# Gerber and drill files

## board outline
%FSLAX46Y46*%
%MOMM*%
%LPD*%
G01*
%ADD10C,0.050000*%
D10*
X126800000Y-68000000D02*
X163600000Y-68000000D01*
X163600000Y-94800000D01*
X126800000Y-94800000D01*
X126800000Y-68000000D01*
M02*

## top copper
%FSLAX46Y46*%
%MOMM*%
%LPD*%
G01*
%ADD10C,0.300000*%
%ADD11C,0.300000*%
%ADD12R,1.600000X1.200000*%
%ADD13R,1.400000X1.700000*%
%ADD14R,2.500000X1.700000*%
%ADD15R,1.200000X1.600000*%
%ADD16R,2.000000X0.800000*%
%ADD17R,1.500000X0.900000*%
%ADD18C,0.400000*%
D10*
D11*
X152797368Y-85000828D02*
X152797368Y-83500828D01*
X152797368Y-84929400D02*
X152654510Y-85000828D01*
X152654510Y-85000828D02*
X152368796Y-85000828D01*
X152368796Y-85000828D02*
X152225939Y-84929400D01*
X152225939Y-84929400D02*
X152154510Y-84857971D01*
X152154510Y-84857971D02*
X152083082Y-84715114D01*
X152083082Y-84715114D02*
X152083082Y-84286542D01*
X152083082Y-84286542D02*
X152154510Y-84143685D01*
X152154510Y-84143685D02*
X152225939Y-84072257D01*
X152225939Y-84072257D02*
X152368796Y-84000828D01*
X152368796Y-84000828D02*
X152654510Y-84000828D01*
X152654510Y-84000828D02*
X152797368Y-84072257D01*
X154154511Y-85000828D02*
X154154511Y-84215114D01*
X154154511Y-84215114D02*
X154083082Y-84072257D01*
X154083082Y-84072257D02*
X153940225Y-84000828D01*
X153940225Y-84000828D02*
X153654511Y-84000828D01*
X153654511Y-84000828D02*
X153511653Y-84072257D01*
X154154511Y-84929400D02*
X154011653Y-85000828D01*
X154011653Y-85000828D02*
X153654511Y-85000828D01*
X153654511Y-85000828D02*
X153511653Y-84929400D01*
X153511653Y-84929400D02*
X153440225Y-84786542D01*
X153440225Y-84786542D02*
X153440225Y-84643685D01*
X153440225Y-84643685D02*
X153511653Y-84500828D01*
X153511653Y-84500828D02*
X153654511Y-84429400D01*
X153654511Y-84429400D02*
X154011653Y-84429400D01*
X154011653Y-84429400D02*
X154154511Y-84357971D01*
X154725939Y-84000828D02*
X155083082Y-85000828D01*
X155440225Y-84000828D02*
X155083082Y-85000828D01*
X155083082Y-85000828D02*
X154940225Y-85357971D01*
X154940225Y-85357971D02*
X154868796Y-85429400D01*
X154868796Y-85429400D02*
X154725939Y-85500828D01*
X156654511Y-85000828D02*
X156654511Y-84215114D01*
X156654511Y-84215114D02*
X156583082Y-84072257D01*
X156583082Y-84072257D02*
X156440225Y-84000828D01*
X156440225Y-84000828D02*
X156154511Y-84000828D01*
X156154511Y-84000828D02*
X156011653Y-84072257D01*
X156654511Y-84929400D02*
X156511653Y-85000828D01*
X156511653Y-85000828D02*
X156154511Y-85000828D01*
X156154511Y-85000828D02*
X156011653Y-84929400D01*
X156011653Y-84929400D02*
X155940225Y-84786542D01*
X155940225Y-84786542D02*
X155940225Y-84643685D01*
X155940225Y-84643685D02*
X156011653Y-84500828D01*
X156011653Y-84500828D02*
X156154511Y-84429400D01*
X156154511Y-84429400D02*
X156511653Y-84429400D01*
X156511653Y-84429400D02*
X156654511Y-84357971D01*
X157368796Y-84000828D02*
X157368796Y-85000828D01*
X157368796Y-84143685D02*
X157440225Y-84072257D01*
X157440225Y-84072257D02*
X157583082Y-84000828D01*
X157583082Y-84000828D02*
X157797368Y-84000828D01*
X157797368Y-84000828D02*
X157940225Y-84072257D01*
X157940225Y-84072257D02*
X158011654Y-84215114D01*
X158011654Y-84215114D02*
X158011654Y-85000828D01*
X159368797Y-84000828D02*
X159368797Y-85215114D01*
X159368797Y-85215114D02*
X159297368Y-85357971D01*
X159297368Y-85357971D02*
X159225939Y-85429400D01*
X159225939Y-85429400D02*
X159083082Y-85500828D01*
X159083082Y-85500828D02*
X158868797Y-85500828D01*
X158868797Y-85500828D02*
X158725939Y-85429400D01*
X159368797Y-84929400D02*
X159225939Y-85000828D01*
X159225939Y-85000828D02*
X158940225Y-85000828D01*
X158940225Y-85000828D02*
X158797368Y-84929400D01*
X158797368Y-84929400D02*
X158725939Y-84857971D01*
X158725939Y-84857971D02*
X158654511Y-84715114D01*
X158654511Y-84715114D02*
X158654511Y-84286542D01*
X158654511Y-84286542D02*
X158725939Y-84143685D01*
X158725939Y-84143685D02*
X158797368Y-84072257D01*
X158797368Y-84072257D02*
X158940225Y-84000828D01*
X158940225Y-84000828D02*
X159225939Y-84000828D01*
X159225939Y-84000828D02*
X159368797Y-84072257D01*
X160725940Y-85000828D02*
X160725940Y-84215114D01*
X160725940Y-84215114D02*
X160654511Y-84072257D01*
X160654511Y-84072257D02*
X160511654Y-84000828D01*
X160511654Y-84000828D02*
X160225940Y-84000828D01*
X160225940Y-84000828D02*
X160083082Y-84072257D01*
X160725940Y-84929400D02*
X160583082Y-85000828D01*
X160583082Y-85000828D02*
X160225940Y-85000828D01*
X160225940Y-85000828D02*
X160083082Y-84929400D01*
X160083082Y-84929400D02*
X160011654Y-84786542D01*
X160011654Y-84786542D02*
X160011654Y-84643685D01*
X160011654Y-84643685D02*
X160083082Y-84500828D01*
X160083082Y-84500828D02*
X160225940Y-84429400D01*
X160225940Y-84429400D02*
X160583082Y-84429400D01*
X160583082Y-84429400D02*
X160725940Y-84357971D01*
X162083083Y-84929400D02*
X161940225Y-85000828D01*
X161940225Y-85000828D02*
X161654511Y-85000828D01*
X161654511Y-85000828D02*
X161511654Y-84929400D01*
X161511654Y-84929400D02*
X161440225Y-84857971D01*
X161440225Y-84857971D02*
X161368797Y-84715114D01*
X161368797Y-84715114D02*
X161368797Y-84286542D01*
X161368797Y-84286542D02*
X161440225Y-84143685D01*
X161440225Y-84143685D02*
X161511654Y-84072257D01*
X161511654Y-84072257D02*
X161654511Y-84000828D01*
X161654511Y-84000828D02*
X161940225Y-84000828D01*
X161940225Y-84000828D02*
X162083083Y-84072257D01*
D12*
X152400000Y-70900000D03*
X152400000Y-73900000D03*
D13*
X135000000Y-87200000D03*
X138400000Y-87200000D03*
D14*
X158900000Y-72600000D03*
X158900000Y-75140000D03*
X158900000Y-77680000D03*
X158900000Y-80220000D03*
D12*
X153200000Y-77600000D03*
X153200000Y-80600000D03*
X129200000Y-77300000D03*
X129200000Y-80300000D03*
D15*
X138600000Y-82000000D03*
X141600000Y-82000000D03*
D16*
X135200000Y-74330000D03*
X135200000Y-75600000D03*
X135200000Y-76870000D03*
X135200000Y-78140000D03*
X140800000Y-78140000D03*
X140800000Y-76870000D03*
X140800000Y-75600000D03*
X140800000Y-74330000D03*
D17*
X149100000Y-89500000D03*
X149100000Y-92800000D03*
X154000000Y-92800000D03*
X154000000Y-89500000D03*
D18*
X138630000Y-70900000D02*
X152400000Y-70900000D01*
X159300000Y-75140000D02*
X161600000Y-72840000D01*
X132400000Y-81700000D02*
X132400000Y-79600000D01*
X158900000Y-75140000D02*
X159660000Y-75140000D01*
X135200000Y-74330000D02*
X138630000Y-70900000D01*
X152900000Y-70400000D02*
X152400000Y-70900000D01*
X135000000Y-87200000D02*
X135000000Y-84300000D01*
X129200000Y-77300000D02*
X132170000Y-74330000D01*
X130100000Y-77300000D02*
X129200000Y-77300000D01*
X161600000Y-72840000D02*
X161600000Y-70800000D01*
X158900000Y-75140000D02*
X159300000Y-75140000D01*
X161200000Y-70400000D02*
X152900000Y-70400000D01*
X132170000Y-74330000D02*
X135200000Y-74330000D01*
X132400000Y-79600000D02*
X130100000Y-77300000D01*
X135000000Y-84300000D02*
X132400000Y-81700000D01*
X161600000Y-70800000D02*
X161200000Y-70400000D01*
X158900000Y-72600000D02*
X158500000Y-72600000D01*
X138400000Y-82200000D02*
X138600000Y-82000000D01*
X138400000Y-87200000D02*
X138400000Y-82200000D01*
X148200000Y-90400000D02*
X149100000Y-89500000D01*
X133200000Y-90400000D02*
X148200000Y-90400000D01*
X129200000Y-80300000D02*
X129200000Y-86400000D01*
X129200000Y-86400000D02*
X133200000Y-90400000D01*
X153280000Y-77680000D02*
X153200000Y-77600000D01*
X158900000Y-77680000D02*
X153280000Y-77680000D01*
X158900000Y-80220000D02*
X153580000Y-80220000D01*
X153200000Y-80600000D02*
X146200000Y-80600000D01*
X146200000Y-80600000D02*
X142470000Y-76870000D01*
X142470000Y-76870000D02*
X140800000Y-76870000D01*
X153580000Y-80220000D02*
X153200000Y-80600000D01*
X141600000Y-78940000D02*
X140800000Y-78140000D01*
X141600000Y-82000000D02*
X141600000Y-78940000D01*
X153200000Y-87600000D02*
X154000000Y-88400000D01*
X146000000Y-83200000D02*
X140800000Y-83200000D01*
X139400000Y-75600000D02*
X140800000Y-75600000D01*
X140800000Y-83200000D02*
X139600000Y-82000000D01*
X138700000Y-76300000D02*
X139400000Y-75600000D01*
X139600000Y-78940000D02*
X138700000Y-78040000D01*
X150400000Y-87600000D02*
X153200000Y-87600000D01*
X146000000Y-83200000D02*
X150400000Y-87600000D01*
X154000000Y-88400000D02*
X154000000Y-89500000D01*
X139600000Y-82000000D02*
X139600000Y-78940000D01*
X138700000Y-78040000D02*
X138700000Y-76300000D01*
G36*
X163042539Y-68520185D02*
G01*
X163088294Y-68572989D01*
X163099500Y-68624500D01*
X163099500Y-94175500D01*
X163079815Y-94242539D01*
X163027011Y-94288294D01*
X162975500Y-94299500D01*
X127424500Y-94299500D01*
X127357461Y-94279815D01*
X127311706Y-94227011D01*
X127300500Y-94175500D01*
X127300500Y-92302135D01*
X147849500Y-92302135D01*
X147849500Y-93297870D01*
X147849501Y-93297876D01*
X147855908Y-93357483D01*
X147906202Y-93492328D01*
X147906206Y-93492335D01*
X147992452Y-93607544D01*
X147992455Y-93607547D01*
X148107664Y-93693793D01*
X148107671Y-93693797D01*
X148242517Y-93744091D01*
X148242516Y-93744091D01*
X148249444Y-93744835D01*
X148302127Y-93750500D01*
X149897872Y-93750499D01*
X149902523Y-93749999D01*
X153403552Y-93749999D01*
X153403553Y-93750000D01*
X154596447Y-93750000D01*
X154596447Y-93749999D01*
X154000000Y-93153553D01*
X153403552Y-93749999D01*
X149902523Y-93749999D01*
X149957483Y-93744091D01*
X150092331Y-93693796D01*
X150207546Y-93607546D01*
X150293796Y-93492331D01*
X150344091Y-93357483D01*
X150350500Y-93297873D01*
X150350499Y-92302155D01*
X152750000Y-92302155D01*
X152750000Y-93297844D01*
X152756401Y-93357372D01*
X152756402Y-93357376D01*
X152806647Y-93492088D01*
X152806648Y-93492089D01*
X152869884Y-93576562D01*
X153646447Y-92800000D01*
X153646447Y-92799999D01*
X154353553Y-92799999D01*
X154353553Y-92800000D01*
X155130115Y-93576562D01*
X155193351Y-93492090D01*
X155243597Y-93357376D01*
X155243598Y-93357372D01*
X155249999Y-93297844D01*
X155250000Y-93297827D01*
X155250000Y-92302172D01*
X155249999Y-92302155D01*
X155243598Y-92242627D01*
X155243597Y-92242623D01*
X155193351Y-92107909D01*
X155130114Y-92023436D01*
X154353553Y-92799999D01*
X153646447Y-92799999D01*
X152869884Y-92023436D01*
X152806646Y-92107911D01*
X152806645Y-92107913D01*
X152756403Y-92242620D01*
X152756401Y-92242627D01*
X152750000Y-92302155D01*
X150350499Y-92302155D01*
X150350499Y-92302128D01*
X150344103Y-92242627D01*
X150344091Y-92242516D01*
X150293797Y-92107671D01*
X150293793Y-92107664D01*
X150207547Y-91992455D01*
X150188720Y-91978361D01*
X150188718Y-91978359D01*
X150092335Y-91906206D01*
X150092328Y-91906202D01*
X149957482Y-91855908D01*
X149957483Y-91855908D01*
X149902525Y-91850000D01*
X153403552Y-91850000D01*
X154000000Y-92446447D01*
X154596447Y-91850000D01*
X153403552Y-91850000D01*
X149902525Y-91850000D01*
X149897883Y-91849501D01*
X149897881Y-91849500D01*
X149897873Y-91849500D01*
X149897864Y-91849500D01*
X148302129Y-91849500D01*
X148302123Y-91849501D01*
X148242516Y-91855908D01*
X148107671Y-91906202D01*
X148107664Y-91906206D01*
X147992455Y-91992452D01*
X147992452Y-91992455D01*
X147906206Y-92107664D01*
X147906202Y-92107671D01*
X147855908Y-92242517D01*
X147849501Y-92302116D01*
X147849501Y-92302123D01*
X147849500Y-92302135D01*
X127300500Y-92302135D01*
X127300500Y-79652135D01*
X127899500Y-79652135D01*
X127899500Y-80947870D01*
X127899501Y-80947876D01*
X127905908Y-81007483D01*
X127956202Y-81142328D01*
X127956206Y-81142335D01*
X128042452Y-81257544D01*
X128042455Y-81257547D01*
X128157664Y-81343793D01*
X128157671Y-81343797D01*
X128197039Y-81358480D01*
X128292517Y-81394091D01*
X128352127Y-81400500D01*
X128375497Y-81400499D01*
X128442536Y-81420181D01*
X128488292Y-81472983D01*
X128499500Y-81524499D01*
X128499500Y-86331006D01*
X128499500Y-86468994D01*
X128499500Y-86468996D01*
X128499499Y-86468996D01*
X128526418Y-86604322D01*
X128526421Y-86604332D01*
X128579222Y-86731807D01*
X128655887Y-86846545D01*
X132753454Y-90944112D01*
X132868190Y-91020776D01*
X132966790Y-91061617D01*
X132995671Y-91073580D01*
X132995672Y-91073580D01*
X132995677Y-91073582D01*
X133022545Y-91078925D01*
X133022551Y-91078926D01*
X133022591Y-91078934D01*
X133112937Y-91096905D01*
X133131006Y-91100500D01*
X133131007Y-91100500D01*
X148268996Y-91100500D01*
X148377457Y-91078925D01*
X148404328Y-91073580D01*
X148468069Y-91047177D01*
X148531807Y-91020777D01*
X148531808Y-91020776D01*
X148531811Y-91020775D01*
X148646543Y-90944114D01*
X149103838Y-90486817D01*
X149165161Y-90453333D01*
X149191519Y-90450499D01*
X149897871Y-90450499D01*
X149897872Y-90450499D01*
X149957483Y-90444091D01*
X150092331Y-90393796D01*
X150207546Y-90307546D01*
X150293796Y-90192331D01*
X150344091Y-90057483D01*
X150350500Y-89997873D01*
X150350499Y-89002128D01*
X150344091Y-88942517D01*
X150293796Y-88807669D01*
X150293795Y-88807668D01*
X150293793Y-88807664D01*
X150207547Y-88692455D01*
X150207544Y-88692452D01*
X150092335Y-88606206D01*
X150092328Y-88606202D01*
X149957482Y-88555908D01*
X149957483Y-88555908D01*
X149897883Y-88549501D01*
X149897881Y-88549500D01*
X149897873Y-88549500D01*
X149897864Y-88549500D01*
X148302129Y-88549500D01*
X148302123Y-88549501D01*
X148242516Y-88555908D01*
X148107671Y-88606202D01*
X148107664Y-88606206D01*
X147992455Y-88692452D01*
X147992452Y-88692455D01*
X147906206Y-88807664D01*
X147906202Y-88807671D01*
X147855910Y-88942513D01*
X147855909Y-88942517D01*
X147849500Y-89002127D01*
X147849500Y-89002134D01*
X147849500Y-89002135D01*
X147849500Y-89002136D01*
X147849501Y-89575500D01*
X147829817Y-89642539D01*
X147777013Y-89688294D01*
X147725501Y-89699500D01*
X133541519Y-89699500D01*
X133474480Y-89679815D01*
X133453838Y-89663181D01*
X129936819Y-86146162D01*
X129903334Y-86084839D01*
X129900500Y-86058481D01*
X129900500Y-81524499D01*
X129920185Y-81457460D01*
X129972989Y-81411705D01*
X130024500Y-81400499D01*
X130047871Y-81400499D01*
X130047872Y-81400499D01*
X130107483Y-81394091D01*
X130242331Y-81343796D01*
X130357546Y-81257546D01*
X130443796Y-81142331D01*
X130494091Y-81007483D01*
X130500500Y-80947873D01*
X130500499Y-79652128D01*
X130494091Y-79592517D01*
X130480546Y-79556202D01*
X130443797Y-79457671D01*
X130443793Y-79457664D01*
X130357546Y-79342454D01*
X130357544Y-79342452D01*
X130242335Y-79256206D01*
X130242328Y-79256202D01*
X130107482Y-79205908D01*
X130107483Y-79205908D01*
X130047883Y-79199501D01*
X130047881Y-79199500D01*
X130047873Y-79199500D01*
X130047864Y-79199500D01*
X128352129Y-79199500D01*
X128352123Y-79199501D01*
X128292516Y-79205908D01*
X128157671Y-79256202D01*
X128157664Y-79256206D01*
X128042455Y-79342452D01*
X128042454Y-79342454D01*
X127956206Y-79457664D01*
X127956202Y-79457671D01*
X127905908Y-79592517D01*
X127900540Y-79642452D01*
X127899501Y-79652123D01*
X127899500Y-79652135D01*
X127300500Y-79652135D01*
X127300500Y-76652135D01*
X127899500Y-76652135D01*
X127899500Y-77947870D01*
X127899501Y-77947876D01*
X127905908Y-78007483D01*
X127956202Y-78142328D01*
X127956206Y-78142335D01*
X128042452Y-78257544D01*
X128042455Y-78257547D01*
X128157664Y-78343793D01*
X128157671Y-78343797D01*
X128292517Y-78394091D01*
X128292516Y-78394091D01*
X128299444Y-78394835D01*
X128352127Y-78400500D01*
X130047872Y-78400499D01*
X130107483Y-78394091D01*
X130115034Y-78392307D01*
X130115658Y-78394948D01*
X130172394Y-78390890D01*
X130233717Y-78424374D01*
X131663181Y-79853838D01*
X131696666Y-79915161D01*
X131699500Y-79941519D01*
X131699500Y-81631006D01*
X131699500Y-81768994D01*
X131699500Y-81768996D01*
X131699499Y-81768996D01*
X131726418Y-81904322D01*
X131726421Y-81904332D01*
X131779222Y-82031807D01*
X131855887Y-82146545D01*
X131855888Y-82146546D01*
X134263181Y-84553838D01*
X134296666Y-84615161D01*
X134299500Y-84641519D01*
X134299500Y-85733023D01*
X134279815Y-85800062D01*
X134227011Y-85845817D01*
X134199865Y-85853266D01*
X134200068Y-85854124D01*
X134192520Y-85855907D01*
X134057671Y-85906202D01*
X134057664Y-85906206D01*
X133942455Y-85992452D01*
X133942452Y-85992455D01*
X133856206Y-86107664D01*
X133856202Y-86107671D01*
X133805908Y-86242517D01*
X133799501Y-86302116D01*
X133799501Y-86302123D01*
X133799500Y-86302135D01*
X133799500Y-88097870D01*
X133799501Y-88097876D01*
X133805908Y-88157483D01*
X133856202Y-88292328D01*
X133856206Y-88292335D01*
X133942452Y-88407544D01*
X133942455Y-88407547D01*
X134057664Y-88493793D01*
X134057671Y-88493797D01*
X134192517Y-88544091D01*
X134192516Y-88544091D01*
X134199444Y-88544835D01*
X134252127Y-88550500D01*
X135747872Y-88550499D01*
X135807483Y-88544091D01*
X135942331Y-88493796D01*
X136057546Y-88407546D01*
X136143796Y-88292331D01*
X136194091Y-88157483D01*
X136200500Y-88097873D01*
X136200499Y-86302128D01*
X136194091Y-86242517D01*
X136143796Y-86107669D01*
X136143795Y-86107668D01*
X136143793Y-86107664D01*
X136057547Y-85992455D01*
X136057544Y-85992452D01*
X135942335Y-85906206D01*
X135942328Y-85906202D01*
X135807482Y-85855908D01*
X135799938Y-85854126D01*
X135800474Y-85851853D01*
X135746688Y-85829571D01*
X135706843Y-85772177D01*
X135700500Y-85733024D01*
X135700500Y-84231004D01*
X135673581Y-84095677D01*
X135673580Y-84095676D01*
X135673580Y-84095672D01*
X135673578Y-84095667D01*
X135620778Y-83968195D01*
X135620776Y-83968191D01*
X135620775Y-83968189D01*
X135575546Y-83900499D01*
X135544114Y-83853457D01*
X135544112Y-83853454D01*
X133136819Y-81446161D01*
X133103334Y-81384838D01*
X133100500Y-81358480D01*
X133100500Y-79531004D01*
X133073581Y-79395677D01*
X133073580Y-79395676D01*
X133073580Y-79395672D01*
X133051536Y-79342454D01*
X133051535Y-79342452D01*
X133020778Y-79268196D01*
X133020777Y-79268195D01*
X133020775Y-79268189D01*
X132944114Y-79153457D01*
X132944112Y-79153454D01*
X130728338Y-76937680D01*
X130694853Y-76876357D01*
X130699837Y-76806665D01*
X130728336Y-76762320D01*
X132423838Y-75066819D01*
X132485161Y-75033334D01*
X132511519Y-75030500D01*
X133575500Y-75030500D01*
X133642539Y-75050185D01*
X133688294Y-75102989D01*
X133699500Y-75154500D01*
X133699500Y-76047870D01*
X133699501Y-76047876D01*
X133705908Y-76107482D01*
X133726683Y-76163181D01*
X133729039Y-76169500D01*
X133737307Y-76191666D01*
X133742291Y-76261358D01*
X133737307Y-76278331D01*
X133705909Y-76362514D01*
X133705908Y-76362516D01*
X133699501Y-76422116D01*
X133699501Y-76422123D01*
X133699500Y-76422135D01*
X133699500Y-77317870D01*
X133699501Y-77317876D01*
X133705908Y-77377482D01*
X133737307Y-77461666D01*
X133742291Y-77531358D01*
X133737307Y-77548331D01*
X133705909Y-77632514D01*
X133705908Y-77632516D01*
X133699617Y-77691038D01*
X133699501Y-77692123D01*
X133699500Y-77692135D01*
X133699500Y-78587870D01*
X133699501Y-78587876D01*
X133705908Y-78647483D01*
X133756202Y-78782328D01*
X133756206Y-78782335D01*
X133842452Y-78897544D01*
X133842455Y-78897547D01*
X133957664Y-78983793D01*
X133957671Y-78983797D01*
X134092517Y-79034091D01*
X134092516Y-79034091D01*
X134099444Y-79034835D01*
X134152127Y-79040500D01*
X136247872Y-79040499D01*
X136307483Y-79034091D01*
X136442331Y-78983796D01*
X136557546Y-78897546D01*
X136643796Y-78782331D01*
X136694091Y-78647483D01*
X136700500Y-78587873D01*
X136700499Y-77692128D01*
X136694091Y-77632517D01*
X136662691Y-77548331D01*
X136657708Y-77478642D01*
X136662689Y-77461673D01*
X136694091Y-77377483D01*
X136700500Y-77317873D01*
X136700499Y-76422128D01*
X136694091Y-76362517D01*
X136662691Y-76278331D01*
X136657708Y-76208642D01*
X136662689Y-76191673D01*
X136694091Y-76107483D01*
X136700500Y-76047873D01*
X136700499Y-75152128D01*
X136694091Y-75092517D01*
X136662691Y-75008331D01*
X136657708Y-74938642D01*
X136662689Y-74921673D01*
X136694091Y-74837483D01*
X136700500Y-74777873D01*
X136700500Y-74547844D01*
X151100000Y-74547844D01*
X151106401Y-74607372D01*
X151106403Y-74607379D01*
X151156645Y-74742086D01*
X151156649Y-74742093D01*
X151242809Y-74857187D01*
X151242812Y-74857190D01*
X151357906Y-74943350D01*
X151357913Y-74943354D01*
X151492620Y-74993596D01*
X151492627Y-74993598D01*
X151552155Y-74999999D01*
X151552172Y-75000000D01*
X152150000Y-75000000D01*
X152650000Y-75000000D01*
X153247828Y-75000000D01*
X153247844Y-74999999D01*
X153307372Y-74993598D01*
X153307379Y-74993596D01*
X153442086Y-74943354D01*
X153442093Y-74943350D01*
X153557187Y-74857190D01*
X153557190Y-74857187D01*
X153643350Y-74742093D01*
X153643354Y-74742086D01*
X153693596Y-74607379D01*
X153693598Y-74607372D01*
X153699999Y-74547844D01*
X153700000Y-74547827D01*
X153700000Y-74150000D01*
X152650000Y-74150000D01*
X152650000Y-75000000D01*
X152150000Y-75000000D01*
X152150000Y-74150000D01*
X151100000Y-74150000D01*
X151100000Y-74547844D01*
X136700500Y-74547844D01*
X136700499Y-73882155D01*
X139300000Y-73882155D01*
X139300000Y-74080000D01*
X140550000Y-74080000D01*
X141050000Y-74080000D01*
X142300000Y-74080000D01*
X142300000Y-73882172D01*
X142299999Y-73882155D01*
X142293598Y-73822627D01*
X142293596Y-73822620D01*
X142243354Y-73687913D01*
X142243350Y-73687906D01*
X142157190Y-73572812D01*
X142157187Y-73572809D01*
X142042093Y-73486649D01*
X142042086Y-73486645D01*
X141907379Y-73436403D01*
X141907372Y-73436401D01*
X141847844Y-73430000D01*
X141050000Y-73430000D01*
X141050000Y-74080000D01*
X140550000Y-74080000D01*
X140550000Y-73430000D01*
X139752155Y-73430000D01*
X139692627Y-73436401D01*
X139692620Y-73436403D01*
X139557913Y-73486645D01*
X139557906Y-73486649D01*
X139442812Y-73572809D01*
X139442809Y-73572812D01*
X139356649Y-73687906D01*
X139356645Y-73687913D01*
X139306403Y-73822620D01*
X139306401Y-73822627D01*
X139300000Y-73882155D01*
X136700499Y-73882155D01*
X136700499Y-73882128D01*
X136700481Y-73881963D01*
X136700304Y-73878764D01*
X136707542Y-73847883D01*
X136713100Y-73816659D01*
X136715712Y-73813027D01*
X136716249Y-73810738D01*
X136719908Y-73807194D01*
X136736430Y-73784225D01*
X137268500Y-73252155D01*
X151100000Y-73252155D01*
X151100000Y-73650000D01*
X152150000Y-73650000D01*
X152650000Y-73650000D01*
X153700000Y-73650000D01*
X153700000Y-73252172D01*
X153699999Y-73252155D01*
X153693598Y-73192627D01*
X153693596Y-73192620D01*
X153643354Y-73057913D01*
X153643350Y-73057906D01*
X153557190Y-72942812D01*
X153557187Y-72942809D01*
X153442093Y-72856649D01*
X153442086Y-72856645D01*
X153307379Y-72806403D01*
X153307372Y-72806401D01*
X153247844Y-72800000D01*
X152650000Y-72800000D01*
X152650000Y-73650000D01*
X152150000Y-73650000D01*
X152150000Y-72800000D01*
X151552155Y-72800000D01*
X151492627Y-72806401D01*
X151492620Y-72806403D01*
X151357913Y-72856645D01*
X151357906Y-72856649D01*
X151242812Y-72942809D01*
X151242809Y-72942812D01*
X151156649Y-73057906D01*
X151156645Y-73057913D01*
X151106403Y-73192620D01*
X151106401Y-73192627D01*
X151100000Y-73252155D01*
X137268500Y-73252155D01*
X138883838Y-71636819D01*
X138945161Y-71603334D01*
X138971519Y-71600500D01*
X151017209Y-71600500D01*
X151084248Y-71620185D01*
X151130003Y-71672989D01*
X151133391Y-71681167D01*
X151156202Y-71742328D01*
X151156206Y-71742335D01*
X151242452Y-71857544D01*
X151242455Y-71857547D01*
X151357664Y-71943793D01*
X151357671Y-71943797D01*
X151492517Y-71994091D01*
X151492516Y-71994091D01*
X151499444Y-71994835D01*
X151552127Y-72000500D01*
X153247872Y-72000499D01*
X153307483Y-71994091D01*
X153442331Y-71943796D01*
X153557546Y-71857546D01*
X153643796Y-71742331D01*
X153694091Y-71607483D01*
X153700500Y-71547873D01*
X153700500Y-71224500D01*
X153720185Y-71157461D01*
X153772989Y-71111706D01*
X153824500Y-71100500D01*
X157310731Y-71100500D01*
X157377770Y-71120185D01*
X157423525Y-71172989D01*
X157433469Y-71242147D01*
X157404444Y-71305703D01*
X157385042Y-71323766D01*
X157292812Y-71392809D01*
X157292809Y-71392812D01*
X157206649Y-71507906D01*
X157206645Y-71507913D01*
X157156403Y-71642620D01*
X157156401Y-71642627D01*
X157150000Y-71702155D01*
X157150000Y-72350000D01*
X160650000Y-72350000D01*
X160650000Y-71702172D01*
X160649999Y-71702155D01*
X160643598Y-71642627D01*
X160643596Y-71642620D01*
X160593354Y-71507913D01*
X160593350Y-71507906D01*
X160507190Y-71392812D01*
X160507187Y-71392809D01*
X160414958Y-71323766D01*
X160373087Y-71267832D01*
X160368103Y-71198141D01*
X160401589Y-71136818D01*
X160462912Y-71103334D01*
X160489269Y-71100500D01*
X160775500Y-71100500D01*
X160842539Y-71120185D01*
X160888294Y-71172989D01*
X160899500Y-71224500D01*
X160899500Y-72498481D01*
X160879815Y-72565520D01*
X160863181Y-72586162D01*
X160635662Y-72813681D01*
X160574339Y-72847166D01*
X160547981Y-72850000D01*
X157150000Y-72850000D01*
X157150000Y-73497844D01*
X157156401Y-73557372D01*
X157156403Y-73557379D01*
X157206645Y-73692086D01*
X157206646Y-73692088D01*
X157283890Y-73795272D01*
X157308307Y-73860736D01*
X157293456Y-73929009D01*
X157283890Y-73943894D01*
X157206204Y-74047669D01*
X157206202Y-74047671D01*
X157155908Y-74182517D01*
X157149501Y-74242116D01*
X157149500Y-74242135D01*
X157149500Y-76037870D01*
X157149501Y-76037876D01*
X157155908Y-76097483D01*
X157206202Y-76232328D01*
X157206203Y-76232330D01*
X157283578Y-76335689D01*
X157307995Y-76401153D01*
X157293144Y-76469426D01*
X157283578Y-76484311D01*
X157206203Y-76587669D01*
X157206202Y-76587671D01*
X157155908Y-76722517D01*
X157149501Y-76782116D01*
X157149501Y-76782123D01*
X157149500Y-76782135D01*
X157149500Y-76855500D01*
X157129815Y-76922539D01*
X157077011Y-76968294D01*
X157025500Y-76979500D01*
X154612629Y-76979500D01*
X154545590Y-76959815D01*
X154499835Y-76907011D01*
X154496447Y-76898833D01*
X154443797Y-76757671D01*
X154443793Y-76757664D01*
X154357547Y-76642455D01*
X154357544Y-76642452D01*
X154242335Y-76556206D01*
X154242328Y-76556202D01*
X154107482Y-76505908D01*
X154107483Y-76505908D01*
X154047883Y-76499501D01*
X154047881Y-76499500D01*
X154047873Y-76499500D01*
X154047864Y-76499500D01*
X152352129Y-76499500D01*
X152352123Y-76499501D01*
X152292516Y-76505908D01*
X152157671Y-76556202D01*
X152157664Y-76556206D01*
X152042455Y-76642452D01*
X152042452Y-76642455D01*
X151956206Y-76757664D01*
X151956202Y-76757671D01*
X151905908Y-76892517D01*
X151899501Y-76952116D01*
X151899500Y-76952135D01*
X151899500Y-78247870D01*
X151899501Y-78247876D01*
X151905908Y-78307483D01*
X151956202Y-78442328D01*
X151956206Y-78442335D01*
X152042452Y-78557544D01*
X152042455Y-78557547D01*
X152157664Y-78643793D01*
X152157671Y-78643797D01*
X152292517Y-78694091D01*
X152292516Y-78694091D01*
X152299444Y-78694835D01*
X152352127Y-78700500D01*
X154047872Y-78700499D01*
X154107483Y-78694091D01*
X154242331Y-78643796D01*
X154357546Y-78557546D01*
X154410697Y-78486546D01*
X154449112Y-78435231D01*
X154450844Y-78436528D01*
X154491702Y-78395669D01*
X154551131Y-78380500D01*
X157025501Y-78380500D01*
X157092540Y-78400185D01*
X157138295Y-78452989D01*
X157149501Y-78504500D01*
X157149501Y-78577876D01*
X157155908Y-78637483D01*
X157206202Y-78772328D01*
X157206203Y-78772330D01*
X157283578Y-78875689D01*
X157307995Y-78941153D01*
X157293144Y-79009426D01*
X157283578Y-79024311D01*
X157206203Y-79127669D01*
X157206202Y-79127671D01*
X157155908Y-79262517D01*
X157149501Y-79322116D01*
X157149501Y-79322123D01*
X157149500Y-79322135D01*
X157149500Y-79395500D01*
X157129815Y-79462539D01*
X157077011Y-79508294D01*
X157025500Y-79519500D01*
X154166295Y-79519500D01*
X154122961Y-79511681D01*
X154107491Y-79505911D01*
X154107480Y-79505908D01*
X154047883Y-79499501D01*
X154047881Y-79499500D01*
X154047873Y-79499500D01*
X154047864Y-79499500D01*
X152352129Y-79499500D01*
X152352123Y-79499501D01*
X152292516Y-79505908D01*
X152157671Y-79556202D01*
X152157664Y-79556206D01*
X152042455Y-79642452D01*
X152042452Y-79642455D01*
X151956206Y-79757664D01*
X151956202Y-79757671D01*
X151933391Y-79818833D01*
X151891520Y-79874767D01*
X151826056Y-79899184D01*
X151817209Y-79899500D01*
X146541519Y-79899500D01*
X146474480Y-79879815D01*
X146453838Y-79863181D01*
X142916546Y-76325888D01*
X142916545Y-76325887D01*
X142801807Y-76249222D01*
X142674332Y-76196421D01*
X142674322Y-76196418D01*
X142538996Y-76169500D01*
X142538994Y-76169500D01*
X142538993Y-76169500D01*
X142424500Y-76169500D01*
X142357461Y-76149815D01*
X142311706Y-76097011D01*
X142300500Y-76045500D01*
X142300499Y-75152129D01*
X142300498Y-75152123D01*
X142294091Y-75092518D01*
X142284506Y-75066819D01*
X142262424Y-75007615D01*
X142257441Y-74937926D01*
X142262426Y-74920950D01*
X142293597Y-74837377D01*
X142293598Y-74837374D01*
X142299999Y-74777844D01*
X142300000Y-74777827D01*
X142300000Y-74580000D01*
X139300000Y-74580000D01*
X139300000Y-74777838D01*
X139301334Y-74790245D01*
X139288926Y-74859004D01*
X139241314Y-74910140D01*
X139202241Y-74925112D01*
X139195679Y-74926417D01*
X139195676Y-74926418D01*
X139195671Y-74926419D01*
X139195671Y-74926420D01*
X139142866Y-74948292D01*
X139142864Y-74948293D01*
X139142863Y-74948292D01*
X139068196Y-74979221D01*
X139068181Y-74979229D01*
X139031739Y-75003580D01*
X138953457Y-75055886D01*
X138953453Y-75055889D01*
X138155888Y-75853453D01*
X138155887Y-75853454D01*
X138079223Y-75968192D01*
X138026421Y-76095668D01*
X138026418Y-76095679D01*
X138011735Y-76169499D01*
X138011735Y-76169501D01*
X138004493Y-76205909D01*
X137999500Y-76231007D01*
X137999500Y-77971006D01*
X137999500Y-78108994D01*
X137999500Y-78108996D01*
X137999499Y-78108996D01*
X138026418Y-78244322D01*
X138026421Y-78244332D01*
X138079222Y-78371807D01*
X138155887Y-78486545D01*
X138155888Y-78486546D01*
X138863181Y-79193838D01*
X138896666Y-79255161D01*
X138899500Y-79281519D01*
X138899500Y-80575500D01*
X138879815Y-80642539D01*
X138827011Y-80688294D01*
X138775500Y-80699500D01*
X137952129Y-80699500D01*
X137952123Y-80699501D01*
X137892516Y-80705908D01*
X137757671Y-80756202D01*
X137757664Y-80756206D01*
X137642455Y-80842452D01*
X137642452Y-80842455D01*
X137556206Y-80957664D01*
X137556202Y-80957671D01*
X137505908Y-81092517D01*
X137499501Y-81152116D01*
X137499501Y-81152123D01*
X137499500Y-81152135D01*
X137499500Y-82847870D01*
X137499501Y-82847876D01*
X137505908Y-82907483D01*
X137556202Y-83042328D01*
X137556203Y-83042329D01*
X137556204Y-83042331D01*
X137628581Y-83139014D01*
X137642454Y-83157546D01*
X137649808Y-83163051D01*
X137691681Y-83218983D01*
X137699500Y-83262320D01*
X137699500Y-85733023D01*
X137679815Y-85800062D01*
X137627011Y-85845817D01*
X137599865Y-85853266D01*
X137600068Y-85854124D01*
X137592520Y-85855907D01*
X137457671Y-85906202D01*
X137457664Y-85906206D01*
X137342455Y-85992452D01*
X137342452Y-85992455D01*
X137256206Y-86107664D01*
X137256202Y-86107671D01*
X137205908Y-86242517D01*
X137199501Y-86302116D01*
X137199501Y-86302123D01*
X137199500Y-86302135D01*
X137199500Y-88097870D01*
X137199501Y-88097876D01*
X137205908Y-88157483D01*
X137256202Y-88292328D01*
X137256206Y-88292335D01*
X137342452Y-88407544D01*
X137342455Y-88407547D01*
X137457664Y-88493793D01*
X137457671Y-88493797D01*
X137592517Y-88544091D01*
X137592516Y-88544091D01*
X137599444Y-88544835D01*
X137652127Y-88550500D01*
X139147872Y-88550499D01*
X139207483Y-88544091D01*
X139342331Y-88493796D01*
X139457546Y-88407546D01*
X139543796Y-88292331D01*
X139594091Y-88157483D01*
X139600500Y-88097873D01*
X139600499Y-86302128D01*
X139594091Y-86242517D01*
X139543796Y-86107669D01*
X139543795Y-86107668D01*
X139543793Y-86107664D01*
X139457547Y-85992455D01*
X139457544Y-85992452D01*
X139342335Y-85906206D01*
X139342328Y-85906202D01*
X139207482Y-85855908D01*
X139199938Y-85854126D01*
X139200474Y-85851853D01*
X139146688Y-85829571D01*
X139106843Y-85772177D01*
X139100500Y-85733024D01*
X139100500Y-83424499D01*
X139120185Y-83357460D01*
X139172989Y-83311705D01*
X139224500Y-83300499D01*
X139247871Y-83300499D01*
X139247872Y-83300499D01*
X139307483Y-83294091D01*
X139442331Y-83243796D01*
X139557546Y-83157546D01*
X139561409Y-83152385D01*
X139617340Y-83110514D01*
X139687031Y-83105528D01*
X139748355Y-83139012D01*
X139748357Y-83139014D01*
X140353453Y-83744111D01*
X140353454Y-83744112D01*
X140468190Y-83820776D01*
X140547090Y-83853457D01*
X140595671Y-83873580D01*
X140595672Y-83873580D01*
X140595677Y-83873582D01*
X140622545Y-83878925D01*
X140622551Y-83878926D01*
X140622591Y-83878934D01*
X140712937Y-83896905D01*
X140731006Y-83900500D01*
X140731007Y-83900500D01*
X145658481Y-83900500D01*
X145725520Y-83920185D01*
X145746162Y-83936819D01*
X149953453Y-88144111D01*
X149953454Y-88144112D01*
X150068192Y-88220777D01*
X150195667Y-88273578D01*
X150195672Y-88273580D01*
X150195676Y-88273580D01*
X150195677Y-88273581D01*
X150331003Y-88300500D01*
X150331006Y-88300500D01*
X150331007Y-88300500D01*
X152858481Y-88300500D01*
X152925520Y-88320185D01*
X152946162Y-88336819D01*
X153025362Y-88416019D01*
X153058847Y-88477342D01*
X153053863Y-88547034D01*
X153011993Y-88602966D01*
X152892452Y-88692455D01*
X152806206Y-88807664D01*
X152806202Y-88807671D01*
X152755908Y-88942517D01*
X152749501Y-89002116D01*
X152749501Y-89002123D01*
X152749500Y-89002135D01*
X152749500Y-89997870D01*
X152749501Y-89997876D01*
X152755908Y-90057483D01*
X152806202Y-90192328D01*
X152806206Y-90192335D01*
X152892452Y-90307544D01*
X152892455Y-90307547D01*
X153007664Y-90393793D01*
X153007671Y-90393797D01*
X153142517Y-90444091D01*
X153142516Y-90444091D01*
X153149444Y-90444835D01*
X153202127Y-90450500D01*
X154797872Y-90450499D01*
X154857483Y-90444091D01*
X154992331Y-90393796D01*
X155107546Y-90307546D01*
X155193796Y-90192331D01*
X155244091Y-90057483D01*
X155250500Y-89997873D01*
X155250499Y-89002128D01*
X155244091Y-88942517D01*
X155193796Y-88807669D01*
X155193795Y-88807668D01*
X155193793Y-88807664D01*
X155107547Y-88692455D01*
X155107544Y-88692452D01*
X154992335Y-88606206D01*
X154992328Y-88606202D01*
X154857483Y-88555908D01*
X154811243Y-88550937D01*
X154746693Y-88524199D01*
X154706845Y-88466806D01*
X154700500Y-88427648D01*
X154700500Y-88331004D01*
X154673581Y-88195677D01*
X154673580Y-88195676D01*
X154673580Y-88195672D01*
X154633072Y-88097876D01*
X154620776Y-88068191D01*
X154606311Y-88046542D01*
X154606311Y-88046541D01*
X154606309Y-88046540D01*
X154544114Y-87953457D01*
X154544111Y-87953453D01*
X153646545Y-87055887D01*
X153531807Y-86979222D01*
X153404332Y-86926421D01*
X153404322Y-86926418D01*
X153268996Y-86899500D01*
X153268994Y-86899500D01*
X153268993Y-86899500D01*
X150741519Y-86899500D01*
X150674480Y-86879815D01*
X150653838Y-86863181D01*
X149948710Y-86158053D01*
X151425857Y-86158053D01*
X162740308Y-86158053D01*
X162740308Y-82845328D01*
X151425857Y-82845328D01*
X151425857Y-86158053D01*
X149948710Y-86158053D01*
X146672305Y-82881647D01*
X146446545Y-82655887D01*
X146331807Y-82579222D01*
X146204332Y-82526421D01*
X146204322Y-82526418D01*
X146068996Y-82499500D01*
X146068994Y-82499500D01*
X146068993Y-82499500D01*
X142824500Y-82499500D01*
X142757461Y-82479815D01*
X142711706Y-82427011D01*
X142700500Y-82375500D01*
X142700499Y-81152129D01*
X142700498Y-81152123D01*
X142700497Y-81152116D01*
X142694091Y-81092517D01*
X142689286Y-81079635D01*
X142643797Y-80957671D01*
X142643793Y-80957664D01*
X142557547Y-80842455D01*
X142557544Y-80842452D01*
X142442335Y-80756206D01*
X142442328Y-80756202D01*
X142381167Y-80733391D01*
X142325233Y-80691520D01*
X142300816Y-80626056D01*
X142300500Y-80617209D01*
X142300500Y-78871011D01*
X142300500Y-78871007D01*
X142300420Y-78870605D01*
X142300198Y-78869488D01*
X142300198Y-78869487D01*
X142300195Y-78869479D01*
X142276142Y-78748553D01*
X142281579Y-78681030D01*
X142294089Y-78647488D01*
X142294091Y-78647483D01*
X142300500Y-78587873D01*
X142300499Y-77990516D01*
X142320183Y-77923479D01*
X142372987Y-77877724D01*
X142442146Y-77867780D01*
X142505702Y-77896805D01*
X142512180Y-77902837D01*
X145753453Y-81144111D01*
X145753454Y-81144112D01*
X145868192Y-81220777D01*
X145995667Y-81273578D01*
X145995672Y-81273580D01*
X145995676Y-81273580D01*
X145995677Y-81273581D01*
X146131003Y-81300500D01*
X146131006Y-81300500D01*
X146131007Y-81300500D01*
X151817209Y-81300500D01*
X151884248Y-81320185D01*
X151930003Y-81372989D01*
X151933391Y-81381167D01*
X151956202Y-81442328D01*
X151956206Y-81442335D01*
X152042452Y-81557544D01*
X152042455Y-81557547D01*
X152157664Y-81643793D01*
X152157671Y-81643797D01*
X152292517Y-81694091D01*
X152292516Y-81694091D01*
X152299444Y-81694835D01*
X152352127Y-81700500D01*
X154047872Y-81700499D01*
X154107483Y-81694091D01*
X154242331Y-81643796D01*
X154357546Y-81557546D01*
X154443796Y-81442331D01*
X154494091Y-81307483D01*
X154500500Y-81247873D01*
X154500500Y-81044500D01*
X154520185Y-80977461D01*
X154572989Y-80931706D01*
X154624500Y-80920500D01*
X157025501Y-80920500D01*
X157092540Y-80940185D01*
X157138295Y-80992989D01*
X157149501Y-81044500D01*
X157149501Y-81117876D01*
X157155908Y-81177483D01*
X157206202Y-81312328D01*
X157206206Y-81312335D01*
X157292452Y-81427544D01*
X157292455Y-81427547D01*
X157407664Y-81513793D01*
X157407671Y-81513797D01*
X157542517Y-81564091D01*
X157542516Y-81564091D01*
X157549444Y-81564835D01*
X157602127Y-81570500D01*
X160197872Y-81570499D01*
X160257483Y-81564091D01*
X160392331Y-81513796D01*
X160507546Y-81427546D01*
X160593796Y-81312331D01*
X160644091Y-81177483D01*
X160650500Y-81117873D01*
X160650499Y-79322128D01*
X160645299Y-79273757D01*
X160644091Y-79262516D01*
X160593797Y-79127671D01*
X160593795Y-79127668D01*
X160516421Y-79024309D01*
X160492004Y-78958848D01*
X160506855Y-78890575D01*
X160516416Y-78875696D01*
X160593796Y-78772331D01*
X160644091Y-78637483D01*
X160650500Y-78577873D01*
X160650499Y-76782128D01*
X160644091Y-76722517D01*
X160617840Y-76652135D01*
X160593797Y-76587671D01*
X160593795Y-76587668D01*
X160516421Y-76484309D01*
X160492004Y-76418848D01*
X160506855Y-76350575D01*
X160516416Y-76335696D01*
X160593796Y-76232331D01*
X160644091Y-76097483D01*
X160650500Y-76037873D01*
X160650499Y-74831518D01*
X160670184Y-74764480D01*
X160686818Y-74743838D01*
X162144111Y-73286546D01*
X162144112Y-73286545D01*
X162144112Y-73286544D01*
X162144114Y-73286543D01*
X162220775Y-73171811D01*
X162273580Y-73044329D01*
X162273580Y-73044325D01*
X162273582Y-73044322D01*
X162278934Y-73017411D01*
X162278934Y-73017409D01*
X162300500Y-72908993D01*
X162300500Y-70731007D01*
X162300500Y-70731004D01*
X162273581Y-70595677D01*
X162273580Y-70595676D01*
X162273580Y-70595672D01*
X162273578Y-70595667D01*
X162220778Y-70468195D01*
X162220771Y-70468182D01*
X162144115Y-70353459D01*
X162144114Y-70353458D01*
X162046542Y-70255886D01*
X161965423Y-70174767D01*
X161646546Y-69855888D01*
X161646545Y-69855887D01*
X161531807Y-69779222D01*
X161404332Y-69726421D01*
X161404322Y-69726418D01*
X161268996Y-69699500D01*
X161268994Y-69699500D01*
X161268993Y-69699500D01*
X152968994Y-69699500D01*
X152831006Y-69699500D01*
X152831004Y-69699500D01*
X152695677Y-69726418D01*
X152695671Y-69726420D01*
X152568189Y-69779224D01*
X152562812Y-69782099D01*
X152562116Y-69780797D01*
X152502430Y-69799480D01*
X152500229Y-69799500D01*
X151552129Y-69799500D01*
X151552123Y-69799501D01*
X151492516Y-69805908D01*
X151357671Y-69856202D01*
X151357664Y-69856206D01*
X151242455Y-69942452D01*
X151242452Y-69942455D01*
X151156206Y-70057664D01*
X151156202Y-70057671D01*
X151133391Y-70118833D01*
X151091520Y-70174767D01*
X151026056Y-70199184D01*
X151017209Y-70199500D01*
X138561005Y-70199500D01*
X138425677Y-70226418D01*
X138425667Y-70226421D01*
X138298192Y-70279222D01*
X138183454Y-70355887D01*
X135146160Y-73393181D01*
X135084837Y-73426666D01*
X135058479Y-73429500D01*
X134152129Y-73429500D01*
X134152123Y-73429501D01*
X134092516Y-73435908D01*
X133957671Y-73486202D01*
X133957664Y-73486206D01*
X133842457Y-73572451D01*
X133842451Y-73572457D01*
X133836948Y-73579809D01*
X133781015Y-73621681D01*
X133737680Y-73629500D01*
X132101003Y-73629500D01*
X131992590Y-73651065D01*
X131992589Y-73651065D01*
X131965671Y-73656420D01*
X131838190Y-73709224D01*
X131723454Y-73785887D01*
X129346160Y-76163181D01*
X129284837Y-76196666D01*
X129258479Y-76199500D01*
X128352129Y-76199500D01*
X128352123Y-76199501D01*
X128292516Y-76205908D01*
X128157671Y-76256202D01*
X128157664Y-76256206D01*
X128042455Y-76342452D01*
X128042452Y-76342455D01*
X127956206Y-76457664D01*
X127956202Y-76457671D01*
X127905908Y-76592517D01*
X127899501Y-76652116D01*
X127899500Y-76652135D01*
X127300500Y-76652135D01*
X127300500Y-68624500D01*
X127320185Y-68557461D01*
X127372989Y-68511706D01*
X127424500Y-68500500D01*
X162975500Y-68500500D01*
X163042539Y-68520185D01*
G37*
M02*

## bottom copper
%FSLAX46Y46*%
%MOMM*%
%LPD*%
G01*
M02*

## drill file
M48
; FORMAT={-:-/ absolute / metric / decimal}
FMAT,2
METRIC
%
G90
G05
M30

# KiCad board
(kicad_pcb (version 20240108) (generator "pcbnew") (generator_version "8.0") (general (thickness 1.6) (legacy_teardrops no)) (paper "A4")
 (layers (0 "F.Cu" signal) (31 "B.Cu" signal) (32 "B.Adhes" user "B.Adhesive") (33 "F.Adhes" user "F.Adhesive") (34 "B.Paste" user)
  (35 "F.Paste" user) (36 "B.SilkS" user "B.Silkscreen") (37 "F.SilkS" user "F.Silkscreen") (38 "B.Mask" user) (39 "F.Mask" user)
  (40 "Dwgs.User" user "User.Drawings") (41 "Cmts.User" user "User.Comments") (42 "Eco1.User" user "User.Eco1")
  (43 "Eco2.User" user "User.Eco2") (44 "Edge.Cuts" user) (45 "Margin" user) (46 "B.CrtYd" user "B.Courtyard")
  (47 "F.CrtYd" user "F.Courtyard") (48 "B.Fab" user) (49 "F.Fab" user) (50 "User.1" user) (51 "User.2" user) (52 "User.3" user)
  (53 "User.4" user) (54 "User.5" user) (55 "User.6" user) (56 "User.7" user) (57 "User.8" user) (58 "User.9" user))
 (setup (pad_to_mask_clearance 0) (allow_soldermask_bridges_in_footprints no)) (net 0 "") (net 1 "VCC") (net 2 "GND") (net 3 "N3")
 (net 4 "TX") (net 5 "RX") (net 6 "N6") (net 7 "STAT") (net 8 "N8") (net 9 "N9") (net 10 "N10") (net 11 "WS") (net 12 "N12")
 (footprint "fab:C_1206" (layer "F.Cu") (at 152.4 72.4 -90)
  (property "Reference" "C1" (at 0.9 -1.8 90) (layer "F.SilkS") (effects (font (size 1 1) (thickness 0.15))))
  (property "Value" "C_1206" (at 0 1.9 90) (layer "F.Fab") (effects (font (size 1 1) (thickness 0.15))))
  (pad "1" smd rect (at -1.5 0 270) (size 1.2 1.6) (layers "F.Cu" "F.Paste" "F.Mask") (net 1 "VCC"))
  (pad "2" smd rect (at 1.5 0 270) (size 1.2 1.6) (layers "F.Cu" "F.Paste" "F.Mask") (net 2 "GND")))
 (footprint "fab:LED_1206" (layer "F.Cu") (at 136.7 87.2)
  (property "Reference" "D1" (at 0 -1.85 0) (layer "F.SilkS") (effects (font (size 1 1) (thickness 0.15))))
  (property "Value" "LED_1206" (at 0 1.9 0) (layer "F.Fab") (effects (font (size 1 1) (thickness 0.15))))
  (pad "1" smd rect (at -1.7 0) (size 1.4 1.7) (layers "F.Cu" "F.Paste" "F.Mask") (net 1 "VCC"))
  (pad "2" smd rect (at 1.7 0) (size 1.4 1.7) (layers "F.Cu" "F.Paste" "F.Mask") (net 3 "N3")))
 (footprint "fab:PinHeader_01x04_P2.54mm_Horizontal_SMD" (layer "F.Cu") (at 158.9 72.6)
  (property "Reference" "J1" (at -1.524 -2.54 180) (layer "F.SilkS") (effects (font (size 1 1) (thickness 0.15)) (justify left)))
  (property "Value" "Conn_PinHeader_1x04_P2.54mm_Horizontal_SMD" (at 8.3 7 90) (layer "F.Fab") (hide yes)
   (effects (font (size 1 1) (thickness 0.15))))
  (pad "1" smd rect (at 0 0) (size 2.5 1.7) (layers "F.Cu" "F.Paste" "F.Mask") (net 2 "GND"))
  (pad "2" smd rect (at 0 2.54) (size 2.5 1.7) (layers "F.Cu" "F.Paste" "F.Mask") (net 1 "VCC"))
  (pad "3" smd rect (at 0 5.08) (size 2.5 1.7) (layers "F.Cu" "F.Paste" "F.Mask") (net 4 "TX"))
  (pad "4" smd rect (at 0 7.62) (size 2.5 1.7) (layers "F.Cu" "F.Paste" "F.Mask") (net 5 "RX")))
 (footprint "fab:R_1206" (layer "F.Cu") (at 153.2 79.1 -90)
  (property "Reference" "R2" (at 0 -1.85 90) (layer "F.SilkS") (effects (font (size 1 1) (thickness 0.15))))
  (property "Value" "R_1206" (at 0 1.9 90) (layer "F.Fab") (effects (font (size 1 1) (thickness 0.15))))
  (pad "1" smd rect (at -1.5 0 270) (size 1.2 1.6) (layers "F.Cu" "F.Paste" "F.Mask") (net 4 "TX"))
  (pad "2" smd rect (at 1.5 0 270) (size 1.2 1.6) (layers "F.Cu" "F.Paste" "F.Mask") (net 5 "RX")))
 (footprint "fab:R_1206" (layer "F.Cu") (at 129.2 78.8 -90)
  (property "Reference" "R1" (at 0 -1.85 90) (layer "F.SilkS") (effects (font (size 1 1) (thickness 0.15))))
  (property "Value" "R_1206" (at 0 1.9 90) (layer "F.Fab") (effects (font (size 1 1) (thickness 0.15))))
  (pad "1" smd rect (at -1.5 0 270) (size 1.2 1.6) (layers "F.Cu" "F.Paste" "F.Mask") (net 1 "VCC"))
  (pad "2" smd rect (at 1.5 0 270) (size 1.2 1.6) (layers "F.Cu" "F.Paste" "F.Mask") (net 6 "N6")))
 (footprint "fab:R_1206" (layer "F.Cu") (at 140.1 82)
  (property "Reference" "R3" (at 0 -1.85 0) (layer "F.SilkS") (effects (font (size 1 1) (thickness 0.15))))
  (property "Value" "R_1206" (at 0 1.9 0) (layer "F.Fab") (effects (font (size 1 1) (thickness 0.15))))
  (pad "1" smd rect (at -1.5 0) (size 1.2 1.6) (layers "F.Cu" "F.Paste" "F.Mask") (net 3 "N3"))
  (pad "2" smd rect (at 1.5 0) (size 1.2 1.6) (layers "F.Cu" "F.Paste" "F.Mask") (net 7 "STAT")))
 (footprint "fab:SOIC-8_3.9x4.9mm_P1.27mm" (layer "F.Cu") (at 138 76.235)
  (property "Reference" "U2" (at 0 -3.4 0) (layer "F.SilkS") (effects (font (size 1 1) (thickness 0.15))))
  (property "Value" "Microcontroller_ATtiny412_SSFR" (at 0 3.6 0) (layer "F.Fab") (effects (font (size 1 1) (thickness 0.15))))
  (pad "1" smd rect (at -2.8 -1.905) (size 2 0.8) (layers "F.Cu" "F.Paste" "F.Mask") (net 1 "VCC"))
  (pad "2" smd rect (at -2.8 -0.635) (size 2 0.8) (layers "F.Cu" "F.Paste" "F.Mask") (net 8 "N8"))
  (pad "3" smd rect (at -2.8 0.635) (size 2 0.8) (layers "F.Cu" "F.Paste" "F.Mask") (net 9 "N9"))
  (pad "4" smd rect (at -2.8 1.905) (size 2 0.8) (layers "F.Cu" "F.Paste" "F.Mask") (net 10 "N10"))
  (pad "5" smd rect (at 2.8 1.905) (size 2 0.8) (layers "F.Cu" "F.Paste" "F.Mask") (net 7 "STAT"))
  (pad "6" smd rect (at 2.8 0.635) (size 2 0.8) (layers "F.Cu" "F.Paste" "F.Mask") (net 5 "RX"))
  (pad "7" smd rect (at 2.8 -0.635) (size 2 0.8) (layers "F.Cu" "F.Paste" "F.Mask") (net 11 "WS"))
  (pad "8" smd rect (at 2.8 -1.905) (size 2 0.8) (layers "F.Cu" "F.Paste" "F.Mask") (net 2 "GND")))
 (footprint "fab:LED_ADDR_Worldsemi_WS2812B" (layer "F.Cu") (at 151.55 91.15)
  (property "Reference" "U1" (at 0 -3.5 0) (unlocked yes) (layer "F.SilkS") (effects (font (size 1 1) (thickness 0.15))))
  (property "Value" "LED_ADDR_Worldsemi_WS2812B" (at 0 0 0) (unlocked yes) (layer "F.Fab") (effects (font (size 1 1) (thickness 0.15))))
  (pad "1" smd rect (at -2.45 -1.65) (size 1.5 0.9) (layers "F.Cu" "F.Paste" "F.Mask") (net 6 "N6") (thermal_bridge_angle 45))
  (pad "2" smd rect (at -2.45 1.65) (size 1.5 0.9) (layers "F.Cu" "F.Paste" "F.Mask") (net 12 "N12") (thermal_bridge_angle 45))
  (pad "3" smd rect (at 2.45 1.65) (size 1.5 0.9) (layers "F.Cu" "F.Paste" "F.Mask") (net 2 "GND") (thermal_bridge_angle 45))
  (pad "4" smd rect (at 2.45 -1.65) (size 1.5 0.9) (layers "F.Cu" "F.Paste" "F.Mask") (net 11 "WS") (thermal_bridge_angle 45)))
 (gr_rect (start 126.8 68) (end 163.6 94.8) (stroke (width 0.05) (type default)) (fill none) (layer "Edge.Cuts"))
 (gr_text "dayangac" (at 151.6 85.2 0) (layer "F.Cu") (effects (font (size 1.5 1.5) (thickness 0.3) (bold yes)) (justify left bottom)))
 (segment (start 138.63 70.9) (end 152.4 70.9) (width 0.4) (layer "F.Cu") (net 1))
 (segment (start 159.3 75.14) (end 161.6 72.84) (width 0.4) (layer "F.Cu") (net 1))
 (segment (start 132.4 81.7) (end 132.4 79.6) (width 0.4) (layer "F.Cu") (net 1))
 (segment (start 158.9 75.14) (end 159.66 75.14) (width 0.4) (layer "F.Cu") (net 1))
 (segment (start 135.2 74.33) (end 138.63 70.9) (width 0.4) (layer "F.Cu") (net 1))
 (segment (start 152.9 70.4) (end 152.4 70.9) (width 0.4) (layer "F.Cu") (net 1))
 (segment (start 135 87.2) (end 135 84.3) (width 0.4) (layer "F.Cu") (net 1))
 (segment (start 129.2 77.3) (end 132.17 74.33) (width 0.4) (layer "F.Cu") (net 1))
 (segment (start 130.1 77.3) (end 129.2 77.3) (width 0.4) (layer "F.Cu") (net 1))
 (segment (start 161.6 72.84) (end 161.6 70.8) (width 0.4) (layer "F.Cu") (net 1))
 (segment (start 158.9 75.14) (end 159.3 75.14) (width 0.4) (layer "F.Cu") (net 1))
 (segment (start 161.2 70.4) (end 152.9 70.4) (width 0.4) (layer "F.Cu") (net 1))
 (segment (start 132.17 74.33) (end 135.2 74.33) (width 0.4) (layer "F.Cu") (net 1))
 (segment (start 132.4 79.6) (end 130.1 77.3) (width 0.4) (layer "F.Cu") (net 1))
 (segment (start 135 84.3) (end 132.4 81.7) (width 0.4) (layer "F.Cu") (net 1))
 (segment (start 161.6 70.8) (end 161.2 70.4) (width 0.4) (layer "F.Cu") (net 1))
 (segment (start 158.9 72.6) (end 158.5 72.6) (width 0.4) (layer "F.Cu") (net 2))
 (segment (start 138.4 82.2) (end 138.6 82) (width 0.4) (layer "F.Cu") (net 3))
 (segment (start 138.4 87.2) (end 138.4 82.2) (width 0.4) (layer "F.Cu") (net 3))
 (segment (start 148.2 90.4) (end 149.1 89.5) (width 0.4) (layer "F.Cu") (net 6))
 (segment (start 133.2 90.4) (end 148.2 90.4) (width 0.4) (layer "F.Cu") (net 6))
 (segment (start 129.2 80.3) (end 129.2 86.4) (width 0.4) (layer "F.Cu") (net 6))
 (segment (start 129.2 86.4) (end 133.2 90.4) (width 0.4) (layer "F.Cu") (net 6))
 (segment (start 153.28 77.68) (end 153.2 77.6) (width 0.4) (layer "F.Cu") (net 4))
 (segment (start 158.9 77.68) (end 153.28 77.68) (width 0.4) (layer "F.Cu") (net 4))
 (segment (start 158.9 80.22) (end 153.58 80.22) (width 0.4) (layer "F.Cu") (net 5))
 (segment (start 153.2 80.6) (end 146.2 80.6) (width 0.4) (layer "F.Cu") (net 5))
 (segment (start 146.2 80.6) (end 142.47 76.87) (width 0.4) (layer "F.Cu") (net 5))
 (segment (start 142.47 76.87) (end 140.8 76.87) (width 0.4) (layer "F.Cu") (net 5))
 (segment (start 153.58 80.22) (end 153.2 80.6) (width 0.4) (layer "F.Cu") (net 5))
 (segment (start 141.6 78.94) (end 140.8 78.14) (width 0.4) (layer "F.Cu") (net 7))
 (segment (start 141.6 82) (end 141.6 78.94) (width 0.4) (layer "F.Cu") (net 7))
 (segment (start 153.2 87.6) (end 154 88.4) (width 0.4) (layer "F.Cu") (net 11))
 (segment (start 146 83.2) (end 140.8 83.2) (width 0.4) (layer "F.Cu") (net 11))
 (segment (start 139.4 75.6) (end 140.8 75.6) (width 0.4) (layer "F.Cu") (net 11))
 (segment (start 140.8 83.2) (end 139.6 82) (width 0.4) (layer "F.Cu") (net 11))
 (segment (start 138.7 76.3) (end 139.4 75.6) (width 0.4) (layer "F.Cu") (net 11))
 (segment (start 139.6 78.94) (end 138.7 78.04) (width 0.4) (layer "F.Cu") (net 11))
 (segment (start 150.4 87.6) (end 153.2 87.6) (width 0.4) (layer "F.Cu") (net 11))
 (segment (start 146 83.2) (end 150.4 87.6) (width 0.4) (layer "F.Cu") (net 11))
 (segment (start 154 88.4) (end 154 89.5) (width 0.4) (layer "F.Cu") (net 11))
 (segment (start 139.6 82) (end 139.6 78.94) (width 0.4) (layer "F.Cu") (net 11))
 (segment (start 138.7 78.04) (end 138.7 76.3) (width 0.4) (layer "F.Cu") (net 11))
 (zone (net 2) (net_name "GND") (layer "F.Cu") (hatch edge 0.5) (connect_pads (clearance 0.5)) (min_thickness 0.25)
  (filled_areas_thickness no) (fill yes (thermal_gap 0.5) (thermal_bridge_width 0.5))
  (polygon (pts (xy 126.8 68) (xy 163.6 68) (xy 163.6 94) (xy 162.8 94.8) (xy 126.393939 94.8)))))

